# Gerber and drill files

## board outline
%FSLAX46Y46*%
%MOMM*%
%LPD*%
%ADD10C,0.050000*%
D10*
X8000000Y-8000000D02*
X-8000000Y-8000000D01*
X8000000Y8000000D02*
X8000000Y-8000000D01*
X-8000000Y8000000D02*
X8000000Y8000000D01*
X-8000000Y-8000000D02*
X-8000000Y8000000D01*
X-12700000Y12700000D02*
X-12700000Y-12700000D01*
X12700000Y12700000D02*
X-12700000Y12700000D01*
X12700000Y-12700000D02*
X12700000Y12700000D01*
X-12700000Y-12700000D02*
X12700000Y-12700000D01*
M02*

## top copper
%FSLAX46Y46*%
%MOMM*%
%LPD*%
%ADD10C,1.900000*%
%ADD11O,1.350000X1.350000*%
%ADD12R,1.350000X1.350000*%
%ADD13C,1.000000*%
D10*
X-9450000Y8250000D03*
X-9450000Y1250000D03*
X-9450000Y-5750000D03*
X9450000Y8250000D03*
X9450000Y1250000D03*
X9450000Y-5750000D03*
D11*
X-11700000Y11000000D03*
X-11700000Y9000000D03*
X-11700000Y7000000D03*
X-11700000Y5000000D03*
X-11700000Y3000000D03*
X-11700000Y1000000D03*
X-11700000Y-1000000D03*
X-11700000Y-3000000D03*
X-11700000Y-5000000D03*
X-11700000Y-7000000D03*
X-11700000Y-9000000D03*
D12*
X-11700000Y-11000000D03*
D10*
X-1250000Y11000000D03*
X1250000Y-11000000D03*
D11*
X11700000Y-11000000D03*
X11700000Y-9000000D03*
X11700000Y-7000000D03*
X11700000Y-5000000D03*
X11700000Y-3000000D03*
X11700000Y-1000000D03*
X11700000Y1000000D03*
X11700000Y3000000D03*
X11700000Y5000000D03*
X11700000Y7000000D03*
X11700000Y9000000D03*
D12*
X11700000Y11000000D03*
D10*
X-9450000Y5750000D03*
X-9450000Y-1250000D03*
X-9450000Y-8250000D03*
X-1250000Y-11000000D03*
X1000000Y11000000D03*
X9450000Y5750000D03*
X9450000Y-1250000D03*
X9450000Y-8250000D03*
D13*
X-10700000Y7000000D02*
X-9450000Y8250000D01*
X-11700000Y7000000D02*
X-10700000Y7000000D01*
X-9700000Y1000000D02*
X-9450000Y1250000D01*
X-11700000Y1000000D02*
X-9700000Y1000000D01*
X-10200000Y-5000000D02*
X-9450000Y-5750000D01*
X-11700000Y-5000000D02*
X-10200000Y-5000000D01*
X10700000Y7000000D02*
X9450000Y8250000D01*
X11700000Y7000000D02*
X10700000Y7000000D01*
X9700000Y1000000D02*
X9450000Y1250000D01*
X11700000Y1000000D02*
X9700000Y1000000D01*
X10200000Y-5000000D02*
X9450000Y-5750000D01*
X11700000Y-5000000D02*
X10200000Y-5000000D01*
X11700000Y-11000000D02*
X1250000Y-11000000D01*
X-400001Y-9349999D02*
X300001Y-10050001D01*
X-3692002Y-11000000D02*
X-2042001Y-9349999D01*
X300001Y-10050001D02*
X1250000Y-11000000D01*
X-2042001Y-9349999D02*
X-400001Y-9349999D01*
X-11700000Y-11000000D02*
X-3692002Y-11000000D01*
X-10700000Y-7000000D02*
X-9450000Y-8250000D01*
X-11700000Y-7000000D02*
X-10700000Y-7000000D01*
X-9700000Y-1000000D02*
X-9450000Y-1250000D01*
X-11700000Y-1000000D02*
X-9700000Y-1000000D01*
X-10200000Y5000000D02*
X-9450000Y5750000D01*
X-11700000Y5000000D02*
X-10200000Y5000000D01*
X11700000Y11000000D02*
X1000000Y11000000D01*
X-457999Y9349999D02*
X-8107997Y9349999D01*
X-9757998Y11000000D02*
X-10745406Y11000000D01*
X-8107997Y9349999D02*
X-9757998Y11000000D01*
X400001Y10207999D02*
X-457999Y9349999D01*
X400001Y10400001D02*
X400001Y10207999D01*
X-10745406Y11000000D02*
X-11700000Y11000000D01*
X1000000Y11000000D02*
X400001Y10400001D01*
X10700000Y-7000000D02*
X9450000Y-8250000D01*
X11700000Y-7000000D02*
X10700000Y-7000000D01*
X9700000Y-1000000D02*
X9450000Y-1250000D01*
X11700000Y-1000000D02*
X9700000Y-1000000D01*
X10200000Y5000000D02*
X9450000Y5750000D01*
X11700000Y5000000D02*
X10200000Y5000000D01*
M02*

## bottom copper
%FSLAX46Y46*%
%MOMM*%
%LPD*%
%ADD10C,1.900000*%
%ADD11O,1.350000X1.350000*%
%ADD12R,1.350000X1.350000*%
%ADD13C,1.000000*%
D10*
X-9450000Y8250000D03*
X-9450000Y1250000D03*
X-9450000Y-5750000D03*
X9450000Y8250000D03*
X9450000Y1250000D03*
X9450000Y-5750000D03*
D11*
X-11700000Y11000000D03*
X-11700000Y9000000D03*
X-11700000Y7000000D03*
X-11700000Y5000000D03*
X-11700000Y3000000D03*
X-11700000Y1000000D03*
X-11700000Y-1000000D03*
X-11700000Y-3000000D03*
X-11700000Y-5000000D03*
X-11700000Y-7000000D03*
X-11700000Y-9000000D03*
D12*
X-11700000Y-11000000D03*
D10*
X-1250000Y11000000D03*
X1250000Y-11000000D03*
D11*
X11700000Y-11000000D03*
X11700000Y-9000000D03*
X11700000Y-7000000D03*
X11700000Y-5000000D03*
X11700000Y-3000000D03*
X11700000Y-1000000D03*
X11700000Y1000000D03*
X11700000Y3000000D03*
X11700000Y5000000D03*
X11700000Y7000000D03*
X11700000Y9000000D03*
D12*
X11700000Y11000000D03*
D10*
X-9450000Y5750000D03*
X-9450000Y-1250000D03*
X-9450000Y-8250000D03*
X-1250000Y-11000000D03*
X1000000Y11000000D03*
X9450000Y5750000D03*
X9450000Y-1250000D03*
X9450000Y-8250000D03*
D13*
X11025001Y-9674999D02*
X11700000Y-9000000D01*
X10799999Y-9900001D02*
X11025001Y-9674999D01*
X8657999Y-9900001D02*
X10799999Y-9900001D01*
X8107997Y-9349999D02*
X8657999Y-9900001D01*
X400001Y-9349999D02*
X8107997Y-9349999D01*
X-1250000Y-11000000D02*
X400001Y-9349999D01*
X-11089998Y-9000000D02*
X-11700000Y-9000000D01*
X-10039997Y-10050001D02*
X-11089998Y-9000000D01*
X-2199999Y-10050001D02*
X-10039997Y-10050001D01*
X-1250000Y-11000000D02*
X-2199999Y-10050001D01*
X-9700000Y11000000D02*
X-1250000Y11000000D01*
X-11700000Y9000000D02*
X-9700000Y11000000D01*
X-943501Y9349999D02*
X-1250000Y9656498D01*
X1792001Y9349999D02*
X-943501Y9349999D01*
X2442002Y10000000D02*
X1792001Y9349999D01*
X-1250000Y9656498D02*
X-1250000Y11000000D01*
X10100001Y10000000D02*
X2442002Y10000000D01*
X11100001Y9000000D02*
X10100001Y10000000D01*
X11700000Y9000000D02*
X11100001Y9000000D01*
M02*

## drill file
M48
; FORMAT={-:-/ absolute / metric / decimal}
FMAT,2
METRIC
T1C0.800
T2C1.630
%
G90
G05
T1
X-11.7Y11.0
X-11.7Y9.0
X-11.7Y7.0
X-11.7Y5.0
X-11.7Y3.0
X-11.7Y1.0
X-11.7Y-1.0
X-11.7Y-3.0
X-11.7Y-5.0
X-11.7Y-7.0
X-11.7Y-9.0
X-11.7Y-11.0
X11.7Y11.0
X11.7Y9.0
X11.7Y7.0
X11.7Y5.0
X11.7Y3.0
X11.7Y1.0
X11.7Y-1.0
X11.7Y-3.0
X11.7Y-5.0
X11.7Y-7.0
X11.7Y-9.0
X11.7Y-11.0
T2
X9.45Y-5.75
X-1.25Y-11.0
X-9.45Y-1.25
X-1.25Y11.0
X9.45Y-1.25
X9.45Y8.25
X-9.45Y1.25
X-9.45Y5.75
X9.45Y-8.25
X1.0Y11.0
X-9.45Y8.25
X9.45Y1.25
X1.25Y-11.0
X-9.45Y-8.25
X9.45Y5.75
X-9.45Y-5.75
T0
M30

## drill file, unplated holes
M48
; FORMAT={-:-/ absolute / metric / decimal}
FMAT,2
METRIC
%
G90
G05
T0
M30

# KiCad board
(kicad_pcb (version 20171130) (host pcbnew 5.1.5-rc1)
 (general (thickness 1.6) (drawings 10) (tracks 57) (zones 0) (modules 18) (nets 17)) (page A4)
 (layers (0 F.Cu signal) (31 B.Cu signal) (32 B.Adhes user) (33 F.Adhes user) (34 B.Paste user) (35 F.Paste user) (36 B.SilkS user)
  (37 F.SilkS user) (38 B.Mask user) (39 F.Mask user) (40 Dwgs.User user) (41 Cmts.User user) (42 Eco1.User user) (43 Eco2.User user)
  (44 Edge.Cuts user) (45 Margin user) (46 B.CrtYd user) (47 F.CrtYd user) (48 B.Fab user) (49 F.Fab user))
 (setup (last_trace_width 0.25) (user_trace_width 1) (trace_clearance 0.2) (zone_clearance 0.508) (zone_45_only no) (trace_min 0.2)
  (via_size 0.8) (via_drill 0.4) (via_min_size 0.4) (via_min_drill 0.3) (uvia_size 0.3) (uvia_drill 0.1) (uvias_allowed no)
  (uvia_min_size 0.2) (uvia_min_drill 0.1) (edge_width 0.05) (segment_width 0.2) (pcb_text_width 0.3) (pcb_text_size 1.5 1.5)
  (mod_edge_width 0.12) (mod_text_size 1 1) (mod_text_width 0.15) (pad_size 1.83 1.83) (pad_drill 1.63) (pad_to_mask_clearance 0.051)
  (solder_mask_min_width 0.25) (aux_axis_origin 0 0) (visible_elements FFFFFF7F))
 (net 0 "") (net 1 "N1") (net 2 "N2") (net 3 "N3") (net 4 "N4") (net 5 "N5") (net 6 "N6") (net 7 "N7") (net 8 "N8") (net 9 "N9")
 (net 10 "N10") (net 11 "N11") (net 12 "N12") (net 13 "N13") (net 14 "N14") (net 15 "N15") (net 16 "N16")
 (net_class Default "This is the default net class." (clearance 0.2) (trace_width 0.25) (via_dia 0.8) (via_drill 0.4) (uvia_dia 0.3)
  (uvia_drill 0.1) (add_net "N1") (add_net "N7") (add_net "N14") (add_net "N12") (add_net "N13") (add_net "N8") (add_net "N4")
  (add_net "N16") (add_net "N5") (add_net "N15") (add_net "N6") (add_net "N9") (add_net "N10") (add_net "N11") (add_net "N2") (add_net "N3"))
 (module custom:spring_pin (layer F.Cu) (at -9.45 -8.25 90)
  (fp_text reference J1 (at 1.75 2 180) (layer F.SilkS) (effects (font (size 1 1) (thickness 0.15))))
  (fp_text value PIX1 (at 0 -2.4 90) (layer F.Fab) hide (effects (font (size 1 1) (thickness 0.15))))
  (pad 1 thru_hole circle (at 0 0 90) (size 1.9 1.9) (drill 1.63) (layers *.Cu *.Mask) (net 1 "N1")))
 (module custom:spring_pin (layer F.Cu) (at -9.45 -1.25 90)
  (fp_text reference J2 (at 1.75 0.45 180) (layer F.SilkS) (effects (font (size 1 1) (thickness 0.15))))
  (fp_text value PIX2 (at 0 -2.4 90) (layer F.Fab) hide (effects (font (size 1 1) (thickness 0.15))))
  (pad 1 thru_hole circle (at 0 0 90) (size 1.9 1.9) (drill 1.63) (layers *.Cu *.Mask) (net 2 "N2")))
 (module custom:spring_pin (layer F.Cu) (at -9.45 5.75 90)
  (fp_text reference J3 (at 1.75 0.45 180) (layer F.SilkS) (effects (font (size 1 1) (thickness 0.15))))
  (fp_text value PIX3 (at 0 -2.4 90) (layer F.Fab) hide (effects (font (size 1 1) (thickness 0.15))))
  (pad 1 thru_hole circle (at 0 0 90) (size 1.9 1.9) (drill 1.63) (layers *.Cu *.Mask) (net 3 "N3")))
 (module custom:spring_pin (layer F.Cu) (at 9.45 -8.25 90)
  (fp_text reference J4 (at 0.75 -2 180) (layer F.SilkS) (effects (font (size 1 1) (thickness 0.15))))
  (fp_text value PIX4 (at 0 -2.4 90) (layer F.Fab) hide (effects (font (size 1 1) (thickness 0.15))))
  (pad 1 thru_hole circle (at 0 0 90) (size 1.9 1.9) (drill 1.63) (layers *.Cu *.Mask) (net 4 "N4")))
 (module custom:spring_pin (layer F.Cu) (at 9.45 -1.25 90)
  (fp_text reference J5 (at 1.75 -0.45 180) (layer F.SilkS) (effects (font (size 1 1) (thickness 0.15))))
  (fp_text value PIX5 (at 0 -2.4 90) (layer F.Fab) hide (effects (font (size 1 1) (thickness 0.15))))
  (pad 1 thru_hole circle (at 0 0 90) (size 1.9 1.9) (drill 1.63) (layers *.Cu *.Mask) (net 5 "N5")))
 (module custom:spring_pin (layer F.Cu) (at 9.45 5.75 90)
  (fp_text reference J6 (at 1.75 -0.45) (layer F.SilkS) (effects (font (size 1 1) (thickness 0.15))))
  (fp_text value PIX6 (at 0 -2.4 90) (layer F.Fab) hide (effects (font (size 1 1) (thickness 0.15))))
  (pad 1 thru_hole circle (at 0 0 90) (size 1.9 1.9) (drill 1.63) (layers *.Cu *.Mask) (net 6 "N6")))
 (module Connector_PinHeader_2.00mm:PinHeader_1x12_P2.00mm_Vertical (layer B.Cu) (at -11.7 11)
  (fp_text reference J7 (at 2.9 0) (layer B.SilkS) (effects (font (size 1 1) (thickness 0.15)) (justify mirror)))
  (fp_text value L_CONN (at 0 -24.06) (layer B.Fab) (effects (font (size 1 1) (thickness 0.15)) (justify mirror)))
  (pad 12 thru_hole oval (at 0 -22) (size 1.35 1.35) (drill 0.8) (layers *.Cu *.Mask) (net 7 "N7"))
  (pad 11 thru_hole oval (at 0 -20) (size 1.35 1.35) (drill 0.8) (layers *.Cu *.Mask) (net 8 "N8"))
  (pad 10 thru_hole oval (at 0 -18) (size 1.35 1.35) (drill 0.8) (layers *.Cu *.Mask) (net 1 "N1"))
  (pad 9 thru_hole oval (at 0 -16) (size 1.35 1.35) (drill 0.8) (layers *.Cu *.Mask) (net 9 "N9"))
  (pad 8 thru_hole oval (at 0 -14) (size 1.35 1.35) (drill 0.8) (layers *.Cu *.Mask))
  (pad 7 thru_hole oval (at 0 -12) (size 1.35 1.35) (drill 0.8) (layers *.Cu *.Mask) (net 2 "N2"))
  (pad 6 thru_hole oval (at 0 -10) (size 1.35 1.35) (drill 0.8) (layers *.Cu *.Mask) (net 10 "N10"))
  (pad 5 thru_hole oval (at 0 -8) (size 1.35 1.35) (drill 0.8) (layers *.Cu *.Mask))
  (pad 4 thru_hole oval (at 0 -6) (size 1.35 1.35) (drill 0.8) (layers *.Cu *.Mask) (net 3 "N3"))
  (pad 3 thru_hole oval (at 0 -4) (size 1.35 1.35) (drill 0.8) (layers *.Cu *.Mask) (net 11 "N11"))
  (pad 2 thru_hole oval (at 0 -2) (size 1.35 1.35) (drill 0.8) (layers *.Cu *.Mask) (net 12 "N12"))
  (pad 1 thru_hole rect (at 0 0) (size 1.35 1.35) (drill 0.8) (layers *.Cu *.Mask) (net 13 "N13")))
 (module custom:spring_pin (layer F.Cu) (at -1.25 -11 90)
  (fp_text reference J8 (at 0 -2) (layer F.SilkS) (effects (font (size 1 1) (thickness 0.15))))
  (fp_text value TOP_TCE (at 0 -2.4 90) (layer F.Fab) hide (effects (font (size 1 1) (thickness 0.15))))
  (pad 1 thru_hole circle (at 0 0 90) (size 1.9 1.9) (drill 1.63) (layers *.Cu *.Mask) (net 8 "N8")))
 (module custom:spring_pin (layer F.Cu) (at 1.25 11 90)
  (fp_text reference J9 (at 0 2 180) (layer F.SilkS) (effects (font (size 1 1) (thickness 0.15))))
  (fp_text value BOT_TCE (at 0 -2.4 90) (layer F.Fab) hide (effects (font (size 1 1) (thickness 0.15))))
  (pad 1 thru_hole circle (at 0 0 90) (size 1.9 1.9) (drill 1.63) (layers *.Cu *.Mask) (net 13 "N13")))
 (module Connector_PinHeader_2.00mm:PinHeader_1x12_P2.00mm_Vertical (layer B.Cu) (at 11.7 -11 180)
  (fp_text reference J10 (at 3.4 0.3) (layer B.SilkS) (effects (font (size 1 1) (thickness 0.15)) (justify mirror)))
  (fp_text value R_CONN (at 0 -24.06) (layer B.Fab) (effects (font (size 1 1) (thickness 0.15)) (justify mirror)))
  (pad 12 thru_hole oval (at 0 -22 180) (size 1.35 1.35) (drill 0.8) (layers *.Cu *.Mask) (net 13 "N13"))
  (pad 11 thru_hole oval (at 0 -20 180) (size 1.35 1.35) (drill 0.8) (layers *.Cu *.Mask) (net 12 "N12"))
  (pad 10 thru_hole oval (at 0 -18 180) (size 1.35 1.35) (drill 0.8) (layers *.Cu *.Mask) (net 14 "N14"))
  (pad 9 thru_hole oval (at 0 -16 180) (size 1.35 1.35) (drill 0.8) (layers *.Cu *.Mask) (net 6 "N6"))
  (pad 8 thru_hole oval (at 0 -14 180) (size 1.35 1.35) (drill 0.8) (layers *.Cu *.Mask))
  (pad 7 thru_hole oval (at 0 -12 180) (size 1.35 1.35) (drill 0.8) (layers *.Cu *.Mask) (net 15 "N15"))
  (pad 6 thru_hole oval (at 0 -10 180) (size 1.35 1.35) (drill 0.8) (layers *.Cu *.Mask) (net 5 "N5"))
  (pad 5 thru_hole oval (at 0 -8 180) (size 1.35 1.35) (drill 0.8) (layers *.Cu *.Mask))
  (pad 4 thru_hole oval (at 0 -6 180) (size 1.35 1.35) (drill 0.8) (layers *.Cu *.Mask) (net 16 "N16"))
  (pad 3 thru_hole oval (at 0 -4 180) (size 1.35 1.35) (drill 0.8) (layers *.Cu *.Mask) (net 4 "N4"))
  (pad 2 thru_hole oval (at 0 -2 180) (size 1.35 1.35) (drill 0.8) (layers *.Cu *.Mask) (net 8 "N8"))
  (pad 1 thru_hole rect (at 0 0 180) (size 1.35 1.35) (drill 0.8) (layers *.Cu *.Mask) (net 7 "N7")))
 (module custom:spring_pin (layer F.Cu) (at -9.45 -5.75 90)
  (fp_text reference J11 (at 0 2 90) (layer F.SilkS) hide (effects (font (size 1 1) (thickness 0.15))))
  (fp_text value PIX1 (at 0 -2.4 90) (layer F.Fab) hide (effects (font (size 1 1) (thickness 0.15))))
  (pad 1 thru_hole circle (at 0 0 90) (size 1.9 1.9) (drill 1.63) (layers *.Cu *.Mask) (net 9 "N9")))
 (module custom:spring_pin (layer F.Cu) (at -9.45 1.25 90)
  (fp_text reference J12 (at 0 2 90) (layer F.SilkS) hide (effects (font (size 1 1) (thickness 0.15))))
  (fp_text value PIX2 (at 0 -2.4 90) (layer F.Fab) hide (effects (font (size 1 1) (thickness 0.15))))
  (pad 1 thru_hole circle (at 0 0 90) (size 1.9 1.9) (drill 1.63) (layers *.Cu *.Mask) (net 10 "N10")))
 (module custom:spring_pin (layer F.Cu) (at -9.45 8.25 90)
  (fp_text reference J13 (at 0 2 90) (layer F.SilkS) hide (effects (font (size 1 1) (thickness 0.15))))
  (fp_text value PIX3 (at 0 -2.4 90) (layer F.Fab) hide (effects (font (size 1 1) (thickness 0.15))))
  (pad 1 thru_hole circle (at 0 0 90) (size 1.9 1.9) (drill 1.63) (layers *.Cu *.Mask) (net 11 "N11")))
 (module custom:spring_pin (layer F.Cu) (at -1.25 11 90)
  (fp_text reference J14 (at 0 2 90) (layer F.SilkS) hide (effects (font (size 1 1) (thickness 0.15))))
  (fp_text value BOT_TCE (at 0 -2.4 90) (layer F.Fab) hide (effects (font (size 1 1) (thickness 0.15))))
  (pad 1 thru_hole circle (at 0 0 90) (size 1.9 1.9) (drill 1.63) (layers *.Cu *.Mask) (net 12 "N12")))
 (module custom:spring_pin (layer F.Cu) (at 1 -11 90)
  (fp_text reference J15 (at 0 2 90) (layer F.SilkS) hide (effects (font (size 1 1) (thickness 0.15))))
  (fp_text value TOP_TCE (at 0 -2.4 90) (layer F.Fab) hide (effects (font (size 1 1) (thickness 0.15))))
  (pad 1 thru_hole circle (at 0 0 90) (size 1.9 1.9) (drill 1.63) (layers *.Cu *.Mask) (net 7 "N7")))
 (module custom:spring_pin (layer F.Cu) (at 9.45 -5.75 90)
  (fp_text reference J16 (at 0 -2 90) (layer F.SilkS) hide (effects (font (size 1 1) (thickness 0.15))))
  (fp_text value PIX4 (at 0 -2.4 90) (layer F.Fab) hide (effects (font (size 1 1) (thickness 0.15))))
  (pad 1 thru_hole circle (at 0 0 90) (size 1.9 1.9) (drill 1.63) (layers *.Cu *.Mask) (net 16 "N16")))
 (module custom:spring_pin (layer F.Cu) (at 9.45 1.25 90)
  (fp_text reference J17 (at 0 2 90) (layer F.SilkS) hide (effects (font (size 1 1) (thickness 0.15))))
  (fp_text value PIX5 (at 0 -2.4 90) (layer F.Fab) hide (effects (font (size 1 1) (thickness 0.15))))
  (pad 1 thru_hole circle (at 0 0 90) (size 1.9 1.9) (drill 1.63) (layers *.Cu *.Mask) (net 15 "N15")))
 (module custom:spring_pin (layer F.Cu) (at 9.45 8.25 90)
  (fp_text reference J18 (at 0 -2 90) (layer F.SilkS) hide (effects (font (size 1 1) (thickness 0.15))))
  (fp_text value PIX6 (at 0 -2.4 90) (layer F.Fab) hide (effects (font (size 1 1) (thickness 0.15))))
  (pad 1 thru_hole circle (at 0 0 90) (size 1.9 1.9) (drill 1.63) (layers *.Cu *.Mask) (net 14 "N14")))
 (gr_line (start 8 8) (end -8 8) (layer Edge.Cuts) (width 0.05))
 (gr_line (start 8 -8) (end 8 8) (layer Edge.Cuts) (width 0.05))
 (gr_line (start -8 -8) (end 8 -8) (layer Edge.Cuts) (width 0.05))
 (gr_line (start -8 8) (end -8 -8) (layer Edge.Cuts) (width 0.05))
 (gr_line (start -12.7 -12.7) (end -12.7 12.7) (layer Edge.Cuts) (width 0.05))
 (gr_line (start 12.7 -12.7) (end -12.7 -12.7) (layer Edge.Cuts) (width 0.05))
 (gr_line (start 12.7 12.7) (end 12.7 -12.7) (layer Edge.Cuts) (width 0.05))
 (gr_line (start -12.7 12.7) (end 12.7 12.7) (layer Edge.Cuts) (width 0.05))
 (segment (start -10.7 -7) (end -9.45 -8.25) (width 1) (layer F.Cu) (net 1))
 (segment (start -11.7 -7) (end -10.7 -7) (width 1) (layer F.Cu) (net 1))
 (segment (start -9.7 -1) (end -9.45 -1.25) (width 1) (layer F.Cu) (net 2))
 (segment (start -11.7 -1) (end -9.7 -1) (width 1) (layer F.Cu) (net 2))
 (segment (start -10.2 5) (end -9.45 5.75) (width 1) (layer F.Cu) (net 3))
 (segment (start -11.7 5) (end -10.2 5) (width 1) (layer F.Cu) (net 3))
 (segment (start 10.7 -7) (end 9.45 -8.25) (width 1) (layer F.Cu) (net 4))
 (segment (start 11.7 -7) (end 10.7 -7) (width 1) (layer F.Cu) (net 4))
 (segment (start 9.7 -1) (end 9.45 -1.25) (width 1) (layer F.Cu) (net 5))
 (segment (start 11.7 -1) (end 9.7 -1) (width 1) (layer F.Cu) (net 5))
 (segment (start 10.2 5) (end 9.45 5.75) (width 1) (layer F.Cu) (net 6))
 (segment (start 11.7 5) (end 10.2 5) (width 1) (layer F.Cu) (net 6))
 (segment (start 11.7 11) (end 1.25 11) (width 1) (layer F.Cu) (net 13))
 (segment (start -0.400001 9.349999) (end 0.300001 10.050001) (width 1) (layer F.Cu) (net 13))
 (segment (start -3.692002 11) (end -2.042001 9.349999) (width 1) (layer F.Cu) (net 13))
 (segment (start 0.300001 10.050001) (end 1.25 11) (width 1) (layer F.Cu) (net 13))
 (segment (start -2.042001 9.349999) (end -0.400001 9.349999) (width 1) (layer F.Cu) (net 13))
 (segment (start -11.7 11) (end -3.692002 11) (width 1) (layer F.Cu) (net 13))
 (segment (start 11.025001 9.674999) (end 11.7 9) (width 1) (layer B.Cu) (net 12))
 (segment (start 10.799999 9.900001) (end 11.025001 9.674999) (width 1) (layer B.Cu) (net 12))
 (segment (start 8.657999 9.900001) (end 10.799999 9.900001) (width 1) (layer B.Cu) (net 12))
 (segment (start 8.107997 9.349999) (end 8.657999 9.900001) (width 1) (layer B.Cu) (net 12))
 (segment (start 0.400001 9.349999) (end 8.107997 9.349999) (width 1) (layer B.Cu) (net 12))
 (segment (start -1.25 11) (end 0.400001 9.349999) (width 1) (layer B.Cu) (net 12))
 (segment (start -11.089998 9) (end -11.7 9) (width 1) (layer B.Cu) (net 12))
 (segment (start -10.039997 10.050001) (end -11.089998 9) (width 1) (layer B.Cu) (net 12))
 (segment (start -2.199999 10.050001) (end -10.039997 10.050001) (width 1) (layer B.Cu) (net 12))
 (segment (start -1.25 11) (end -2.199999 10.050001) (width 1) (layer B.Cu) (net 12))
 (segment (start -10.7 7) (end -9.45 8.25) (width 1) (layer F.Cu) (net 11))
 (segment (start -11.7 7) (end -10.7 7) (width 1) (layer F.Cu) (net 11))
 (segment (start -9.7 1) (end -9.45 1.25) (width 1) (layer F.Cu) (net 10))
 (segment (start -11.7 1) (end -9.7 1) (width 1) (layer F.Cu) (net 10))
 (segment (start -10.2 -5) (end -9.45 -5.75) (width 1) (layer F.Cu) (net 9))
 (segment (start -11.7 -5) (end -10.2 -5) (width 1) (layer F.Cu) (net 9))
 (segment (start -9.7 -11) (end -1.25 -11) (width 1) (layer B.Cu) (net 8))
 (segment (start -11.7 -9) (end -9.7 -11) (width 1) (layer B.Cu) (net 8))
 (segment (start -0.943501 -9.349999) (end -1.25 -9.656498) (width 1) (layer B.Cu) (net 8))
 (segment (start 1.792001 -9.349999) (end -0.943501 -9.349999) (width 1) (layer B.Cu) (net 8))
 (segment (start 2.442002 -10) (end 1.792001 -9.349999) (width 1) (layer B.Cu) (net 8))
 (segment (start -1.25 -9.656498) (end -1.25 -11) (width 1) (layer B.Cu) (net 8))
 (segment (start 10.100001 -10) (end 2.442002 -10) (width 1) (layer B.Cu) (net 8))
 (segment (start 11.100001 -9) (end 10.100001 -10) (width 1) (layer B.Cu) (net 8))
 (segment (start 11.7 -9) (end 11.100001 -9) (width 1) (layer B.Cu) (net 8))
 (segment (start 11.7 -11) (end 1 -11) (width 1) (layer F.Cu) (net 7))
 (segment (start -0.457999 -9.349999) (end -8.107997 -9.349999) (width 1) (layer F.Cu) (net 7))
 (segment (start -9.757998 -11) (end -10.745406 -11) (width 1) (layer F.Cu) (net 7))
 (segment (start -8.107997 -9.349999) (end -9.757998 -11) (width 1) (layer F.Cu) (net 7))
 (segment (start 0.400001 -10.207999) (end -0.457999 -9.349999) (width 1) (layer F.Cu) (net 7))
 (segment (start 0.400001 -10.400001) (end 0.400001 -10.207999) (width 1) (layer F.Cu) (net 7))
 (segment (start -10.745406 -11) (end -11.7 -11) (width 1) (layer F.Cu) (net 7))
 (segment (start 1 -11) (end 0.400001 -10.400001) (width 1) (layer F.Cu) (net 7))
 (segment (start 10.7 7) (end 9.45 8.25) (width 1) (layer F.Cu) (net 14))
 (segment (start 11.7 7) (end 10.7 7) (width 1) (layer F.Cu) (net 14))
 (segment (start 9.7 1) (end 9.45 1.25) (width 1) (layer F.Cu) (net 15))
 (segment (start 11.7 1) (end 9.7 1) (width 1) (layer F.Cu) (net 15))
 (segment (start 10.2 -5) (end 9.45 -5.75) (width 1) (layer F.Cu) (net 16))
 (segment (start 11.7 -5) (end 10.2 -5) (width 1) (layer F.Cu) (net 16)))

